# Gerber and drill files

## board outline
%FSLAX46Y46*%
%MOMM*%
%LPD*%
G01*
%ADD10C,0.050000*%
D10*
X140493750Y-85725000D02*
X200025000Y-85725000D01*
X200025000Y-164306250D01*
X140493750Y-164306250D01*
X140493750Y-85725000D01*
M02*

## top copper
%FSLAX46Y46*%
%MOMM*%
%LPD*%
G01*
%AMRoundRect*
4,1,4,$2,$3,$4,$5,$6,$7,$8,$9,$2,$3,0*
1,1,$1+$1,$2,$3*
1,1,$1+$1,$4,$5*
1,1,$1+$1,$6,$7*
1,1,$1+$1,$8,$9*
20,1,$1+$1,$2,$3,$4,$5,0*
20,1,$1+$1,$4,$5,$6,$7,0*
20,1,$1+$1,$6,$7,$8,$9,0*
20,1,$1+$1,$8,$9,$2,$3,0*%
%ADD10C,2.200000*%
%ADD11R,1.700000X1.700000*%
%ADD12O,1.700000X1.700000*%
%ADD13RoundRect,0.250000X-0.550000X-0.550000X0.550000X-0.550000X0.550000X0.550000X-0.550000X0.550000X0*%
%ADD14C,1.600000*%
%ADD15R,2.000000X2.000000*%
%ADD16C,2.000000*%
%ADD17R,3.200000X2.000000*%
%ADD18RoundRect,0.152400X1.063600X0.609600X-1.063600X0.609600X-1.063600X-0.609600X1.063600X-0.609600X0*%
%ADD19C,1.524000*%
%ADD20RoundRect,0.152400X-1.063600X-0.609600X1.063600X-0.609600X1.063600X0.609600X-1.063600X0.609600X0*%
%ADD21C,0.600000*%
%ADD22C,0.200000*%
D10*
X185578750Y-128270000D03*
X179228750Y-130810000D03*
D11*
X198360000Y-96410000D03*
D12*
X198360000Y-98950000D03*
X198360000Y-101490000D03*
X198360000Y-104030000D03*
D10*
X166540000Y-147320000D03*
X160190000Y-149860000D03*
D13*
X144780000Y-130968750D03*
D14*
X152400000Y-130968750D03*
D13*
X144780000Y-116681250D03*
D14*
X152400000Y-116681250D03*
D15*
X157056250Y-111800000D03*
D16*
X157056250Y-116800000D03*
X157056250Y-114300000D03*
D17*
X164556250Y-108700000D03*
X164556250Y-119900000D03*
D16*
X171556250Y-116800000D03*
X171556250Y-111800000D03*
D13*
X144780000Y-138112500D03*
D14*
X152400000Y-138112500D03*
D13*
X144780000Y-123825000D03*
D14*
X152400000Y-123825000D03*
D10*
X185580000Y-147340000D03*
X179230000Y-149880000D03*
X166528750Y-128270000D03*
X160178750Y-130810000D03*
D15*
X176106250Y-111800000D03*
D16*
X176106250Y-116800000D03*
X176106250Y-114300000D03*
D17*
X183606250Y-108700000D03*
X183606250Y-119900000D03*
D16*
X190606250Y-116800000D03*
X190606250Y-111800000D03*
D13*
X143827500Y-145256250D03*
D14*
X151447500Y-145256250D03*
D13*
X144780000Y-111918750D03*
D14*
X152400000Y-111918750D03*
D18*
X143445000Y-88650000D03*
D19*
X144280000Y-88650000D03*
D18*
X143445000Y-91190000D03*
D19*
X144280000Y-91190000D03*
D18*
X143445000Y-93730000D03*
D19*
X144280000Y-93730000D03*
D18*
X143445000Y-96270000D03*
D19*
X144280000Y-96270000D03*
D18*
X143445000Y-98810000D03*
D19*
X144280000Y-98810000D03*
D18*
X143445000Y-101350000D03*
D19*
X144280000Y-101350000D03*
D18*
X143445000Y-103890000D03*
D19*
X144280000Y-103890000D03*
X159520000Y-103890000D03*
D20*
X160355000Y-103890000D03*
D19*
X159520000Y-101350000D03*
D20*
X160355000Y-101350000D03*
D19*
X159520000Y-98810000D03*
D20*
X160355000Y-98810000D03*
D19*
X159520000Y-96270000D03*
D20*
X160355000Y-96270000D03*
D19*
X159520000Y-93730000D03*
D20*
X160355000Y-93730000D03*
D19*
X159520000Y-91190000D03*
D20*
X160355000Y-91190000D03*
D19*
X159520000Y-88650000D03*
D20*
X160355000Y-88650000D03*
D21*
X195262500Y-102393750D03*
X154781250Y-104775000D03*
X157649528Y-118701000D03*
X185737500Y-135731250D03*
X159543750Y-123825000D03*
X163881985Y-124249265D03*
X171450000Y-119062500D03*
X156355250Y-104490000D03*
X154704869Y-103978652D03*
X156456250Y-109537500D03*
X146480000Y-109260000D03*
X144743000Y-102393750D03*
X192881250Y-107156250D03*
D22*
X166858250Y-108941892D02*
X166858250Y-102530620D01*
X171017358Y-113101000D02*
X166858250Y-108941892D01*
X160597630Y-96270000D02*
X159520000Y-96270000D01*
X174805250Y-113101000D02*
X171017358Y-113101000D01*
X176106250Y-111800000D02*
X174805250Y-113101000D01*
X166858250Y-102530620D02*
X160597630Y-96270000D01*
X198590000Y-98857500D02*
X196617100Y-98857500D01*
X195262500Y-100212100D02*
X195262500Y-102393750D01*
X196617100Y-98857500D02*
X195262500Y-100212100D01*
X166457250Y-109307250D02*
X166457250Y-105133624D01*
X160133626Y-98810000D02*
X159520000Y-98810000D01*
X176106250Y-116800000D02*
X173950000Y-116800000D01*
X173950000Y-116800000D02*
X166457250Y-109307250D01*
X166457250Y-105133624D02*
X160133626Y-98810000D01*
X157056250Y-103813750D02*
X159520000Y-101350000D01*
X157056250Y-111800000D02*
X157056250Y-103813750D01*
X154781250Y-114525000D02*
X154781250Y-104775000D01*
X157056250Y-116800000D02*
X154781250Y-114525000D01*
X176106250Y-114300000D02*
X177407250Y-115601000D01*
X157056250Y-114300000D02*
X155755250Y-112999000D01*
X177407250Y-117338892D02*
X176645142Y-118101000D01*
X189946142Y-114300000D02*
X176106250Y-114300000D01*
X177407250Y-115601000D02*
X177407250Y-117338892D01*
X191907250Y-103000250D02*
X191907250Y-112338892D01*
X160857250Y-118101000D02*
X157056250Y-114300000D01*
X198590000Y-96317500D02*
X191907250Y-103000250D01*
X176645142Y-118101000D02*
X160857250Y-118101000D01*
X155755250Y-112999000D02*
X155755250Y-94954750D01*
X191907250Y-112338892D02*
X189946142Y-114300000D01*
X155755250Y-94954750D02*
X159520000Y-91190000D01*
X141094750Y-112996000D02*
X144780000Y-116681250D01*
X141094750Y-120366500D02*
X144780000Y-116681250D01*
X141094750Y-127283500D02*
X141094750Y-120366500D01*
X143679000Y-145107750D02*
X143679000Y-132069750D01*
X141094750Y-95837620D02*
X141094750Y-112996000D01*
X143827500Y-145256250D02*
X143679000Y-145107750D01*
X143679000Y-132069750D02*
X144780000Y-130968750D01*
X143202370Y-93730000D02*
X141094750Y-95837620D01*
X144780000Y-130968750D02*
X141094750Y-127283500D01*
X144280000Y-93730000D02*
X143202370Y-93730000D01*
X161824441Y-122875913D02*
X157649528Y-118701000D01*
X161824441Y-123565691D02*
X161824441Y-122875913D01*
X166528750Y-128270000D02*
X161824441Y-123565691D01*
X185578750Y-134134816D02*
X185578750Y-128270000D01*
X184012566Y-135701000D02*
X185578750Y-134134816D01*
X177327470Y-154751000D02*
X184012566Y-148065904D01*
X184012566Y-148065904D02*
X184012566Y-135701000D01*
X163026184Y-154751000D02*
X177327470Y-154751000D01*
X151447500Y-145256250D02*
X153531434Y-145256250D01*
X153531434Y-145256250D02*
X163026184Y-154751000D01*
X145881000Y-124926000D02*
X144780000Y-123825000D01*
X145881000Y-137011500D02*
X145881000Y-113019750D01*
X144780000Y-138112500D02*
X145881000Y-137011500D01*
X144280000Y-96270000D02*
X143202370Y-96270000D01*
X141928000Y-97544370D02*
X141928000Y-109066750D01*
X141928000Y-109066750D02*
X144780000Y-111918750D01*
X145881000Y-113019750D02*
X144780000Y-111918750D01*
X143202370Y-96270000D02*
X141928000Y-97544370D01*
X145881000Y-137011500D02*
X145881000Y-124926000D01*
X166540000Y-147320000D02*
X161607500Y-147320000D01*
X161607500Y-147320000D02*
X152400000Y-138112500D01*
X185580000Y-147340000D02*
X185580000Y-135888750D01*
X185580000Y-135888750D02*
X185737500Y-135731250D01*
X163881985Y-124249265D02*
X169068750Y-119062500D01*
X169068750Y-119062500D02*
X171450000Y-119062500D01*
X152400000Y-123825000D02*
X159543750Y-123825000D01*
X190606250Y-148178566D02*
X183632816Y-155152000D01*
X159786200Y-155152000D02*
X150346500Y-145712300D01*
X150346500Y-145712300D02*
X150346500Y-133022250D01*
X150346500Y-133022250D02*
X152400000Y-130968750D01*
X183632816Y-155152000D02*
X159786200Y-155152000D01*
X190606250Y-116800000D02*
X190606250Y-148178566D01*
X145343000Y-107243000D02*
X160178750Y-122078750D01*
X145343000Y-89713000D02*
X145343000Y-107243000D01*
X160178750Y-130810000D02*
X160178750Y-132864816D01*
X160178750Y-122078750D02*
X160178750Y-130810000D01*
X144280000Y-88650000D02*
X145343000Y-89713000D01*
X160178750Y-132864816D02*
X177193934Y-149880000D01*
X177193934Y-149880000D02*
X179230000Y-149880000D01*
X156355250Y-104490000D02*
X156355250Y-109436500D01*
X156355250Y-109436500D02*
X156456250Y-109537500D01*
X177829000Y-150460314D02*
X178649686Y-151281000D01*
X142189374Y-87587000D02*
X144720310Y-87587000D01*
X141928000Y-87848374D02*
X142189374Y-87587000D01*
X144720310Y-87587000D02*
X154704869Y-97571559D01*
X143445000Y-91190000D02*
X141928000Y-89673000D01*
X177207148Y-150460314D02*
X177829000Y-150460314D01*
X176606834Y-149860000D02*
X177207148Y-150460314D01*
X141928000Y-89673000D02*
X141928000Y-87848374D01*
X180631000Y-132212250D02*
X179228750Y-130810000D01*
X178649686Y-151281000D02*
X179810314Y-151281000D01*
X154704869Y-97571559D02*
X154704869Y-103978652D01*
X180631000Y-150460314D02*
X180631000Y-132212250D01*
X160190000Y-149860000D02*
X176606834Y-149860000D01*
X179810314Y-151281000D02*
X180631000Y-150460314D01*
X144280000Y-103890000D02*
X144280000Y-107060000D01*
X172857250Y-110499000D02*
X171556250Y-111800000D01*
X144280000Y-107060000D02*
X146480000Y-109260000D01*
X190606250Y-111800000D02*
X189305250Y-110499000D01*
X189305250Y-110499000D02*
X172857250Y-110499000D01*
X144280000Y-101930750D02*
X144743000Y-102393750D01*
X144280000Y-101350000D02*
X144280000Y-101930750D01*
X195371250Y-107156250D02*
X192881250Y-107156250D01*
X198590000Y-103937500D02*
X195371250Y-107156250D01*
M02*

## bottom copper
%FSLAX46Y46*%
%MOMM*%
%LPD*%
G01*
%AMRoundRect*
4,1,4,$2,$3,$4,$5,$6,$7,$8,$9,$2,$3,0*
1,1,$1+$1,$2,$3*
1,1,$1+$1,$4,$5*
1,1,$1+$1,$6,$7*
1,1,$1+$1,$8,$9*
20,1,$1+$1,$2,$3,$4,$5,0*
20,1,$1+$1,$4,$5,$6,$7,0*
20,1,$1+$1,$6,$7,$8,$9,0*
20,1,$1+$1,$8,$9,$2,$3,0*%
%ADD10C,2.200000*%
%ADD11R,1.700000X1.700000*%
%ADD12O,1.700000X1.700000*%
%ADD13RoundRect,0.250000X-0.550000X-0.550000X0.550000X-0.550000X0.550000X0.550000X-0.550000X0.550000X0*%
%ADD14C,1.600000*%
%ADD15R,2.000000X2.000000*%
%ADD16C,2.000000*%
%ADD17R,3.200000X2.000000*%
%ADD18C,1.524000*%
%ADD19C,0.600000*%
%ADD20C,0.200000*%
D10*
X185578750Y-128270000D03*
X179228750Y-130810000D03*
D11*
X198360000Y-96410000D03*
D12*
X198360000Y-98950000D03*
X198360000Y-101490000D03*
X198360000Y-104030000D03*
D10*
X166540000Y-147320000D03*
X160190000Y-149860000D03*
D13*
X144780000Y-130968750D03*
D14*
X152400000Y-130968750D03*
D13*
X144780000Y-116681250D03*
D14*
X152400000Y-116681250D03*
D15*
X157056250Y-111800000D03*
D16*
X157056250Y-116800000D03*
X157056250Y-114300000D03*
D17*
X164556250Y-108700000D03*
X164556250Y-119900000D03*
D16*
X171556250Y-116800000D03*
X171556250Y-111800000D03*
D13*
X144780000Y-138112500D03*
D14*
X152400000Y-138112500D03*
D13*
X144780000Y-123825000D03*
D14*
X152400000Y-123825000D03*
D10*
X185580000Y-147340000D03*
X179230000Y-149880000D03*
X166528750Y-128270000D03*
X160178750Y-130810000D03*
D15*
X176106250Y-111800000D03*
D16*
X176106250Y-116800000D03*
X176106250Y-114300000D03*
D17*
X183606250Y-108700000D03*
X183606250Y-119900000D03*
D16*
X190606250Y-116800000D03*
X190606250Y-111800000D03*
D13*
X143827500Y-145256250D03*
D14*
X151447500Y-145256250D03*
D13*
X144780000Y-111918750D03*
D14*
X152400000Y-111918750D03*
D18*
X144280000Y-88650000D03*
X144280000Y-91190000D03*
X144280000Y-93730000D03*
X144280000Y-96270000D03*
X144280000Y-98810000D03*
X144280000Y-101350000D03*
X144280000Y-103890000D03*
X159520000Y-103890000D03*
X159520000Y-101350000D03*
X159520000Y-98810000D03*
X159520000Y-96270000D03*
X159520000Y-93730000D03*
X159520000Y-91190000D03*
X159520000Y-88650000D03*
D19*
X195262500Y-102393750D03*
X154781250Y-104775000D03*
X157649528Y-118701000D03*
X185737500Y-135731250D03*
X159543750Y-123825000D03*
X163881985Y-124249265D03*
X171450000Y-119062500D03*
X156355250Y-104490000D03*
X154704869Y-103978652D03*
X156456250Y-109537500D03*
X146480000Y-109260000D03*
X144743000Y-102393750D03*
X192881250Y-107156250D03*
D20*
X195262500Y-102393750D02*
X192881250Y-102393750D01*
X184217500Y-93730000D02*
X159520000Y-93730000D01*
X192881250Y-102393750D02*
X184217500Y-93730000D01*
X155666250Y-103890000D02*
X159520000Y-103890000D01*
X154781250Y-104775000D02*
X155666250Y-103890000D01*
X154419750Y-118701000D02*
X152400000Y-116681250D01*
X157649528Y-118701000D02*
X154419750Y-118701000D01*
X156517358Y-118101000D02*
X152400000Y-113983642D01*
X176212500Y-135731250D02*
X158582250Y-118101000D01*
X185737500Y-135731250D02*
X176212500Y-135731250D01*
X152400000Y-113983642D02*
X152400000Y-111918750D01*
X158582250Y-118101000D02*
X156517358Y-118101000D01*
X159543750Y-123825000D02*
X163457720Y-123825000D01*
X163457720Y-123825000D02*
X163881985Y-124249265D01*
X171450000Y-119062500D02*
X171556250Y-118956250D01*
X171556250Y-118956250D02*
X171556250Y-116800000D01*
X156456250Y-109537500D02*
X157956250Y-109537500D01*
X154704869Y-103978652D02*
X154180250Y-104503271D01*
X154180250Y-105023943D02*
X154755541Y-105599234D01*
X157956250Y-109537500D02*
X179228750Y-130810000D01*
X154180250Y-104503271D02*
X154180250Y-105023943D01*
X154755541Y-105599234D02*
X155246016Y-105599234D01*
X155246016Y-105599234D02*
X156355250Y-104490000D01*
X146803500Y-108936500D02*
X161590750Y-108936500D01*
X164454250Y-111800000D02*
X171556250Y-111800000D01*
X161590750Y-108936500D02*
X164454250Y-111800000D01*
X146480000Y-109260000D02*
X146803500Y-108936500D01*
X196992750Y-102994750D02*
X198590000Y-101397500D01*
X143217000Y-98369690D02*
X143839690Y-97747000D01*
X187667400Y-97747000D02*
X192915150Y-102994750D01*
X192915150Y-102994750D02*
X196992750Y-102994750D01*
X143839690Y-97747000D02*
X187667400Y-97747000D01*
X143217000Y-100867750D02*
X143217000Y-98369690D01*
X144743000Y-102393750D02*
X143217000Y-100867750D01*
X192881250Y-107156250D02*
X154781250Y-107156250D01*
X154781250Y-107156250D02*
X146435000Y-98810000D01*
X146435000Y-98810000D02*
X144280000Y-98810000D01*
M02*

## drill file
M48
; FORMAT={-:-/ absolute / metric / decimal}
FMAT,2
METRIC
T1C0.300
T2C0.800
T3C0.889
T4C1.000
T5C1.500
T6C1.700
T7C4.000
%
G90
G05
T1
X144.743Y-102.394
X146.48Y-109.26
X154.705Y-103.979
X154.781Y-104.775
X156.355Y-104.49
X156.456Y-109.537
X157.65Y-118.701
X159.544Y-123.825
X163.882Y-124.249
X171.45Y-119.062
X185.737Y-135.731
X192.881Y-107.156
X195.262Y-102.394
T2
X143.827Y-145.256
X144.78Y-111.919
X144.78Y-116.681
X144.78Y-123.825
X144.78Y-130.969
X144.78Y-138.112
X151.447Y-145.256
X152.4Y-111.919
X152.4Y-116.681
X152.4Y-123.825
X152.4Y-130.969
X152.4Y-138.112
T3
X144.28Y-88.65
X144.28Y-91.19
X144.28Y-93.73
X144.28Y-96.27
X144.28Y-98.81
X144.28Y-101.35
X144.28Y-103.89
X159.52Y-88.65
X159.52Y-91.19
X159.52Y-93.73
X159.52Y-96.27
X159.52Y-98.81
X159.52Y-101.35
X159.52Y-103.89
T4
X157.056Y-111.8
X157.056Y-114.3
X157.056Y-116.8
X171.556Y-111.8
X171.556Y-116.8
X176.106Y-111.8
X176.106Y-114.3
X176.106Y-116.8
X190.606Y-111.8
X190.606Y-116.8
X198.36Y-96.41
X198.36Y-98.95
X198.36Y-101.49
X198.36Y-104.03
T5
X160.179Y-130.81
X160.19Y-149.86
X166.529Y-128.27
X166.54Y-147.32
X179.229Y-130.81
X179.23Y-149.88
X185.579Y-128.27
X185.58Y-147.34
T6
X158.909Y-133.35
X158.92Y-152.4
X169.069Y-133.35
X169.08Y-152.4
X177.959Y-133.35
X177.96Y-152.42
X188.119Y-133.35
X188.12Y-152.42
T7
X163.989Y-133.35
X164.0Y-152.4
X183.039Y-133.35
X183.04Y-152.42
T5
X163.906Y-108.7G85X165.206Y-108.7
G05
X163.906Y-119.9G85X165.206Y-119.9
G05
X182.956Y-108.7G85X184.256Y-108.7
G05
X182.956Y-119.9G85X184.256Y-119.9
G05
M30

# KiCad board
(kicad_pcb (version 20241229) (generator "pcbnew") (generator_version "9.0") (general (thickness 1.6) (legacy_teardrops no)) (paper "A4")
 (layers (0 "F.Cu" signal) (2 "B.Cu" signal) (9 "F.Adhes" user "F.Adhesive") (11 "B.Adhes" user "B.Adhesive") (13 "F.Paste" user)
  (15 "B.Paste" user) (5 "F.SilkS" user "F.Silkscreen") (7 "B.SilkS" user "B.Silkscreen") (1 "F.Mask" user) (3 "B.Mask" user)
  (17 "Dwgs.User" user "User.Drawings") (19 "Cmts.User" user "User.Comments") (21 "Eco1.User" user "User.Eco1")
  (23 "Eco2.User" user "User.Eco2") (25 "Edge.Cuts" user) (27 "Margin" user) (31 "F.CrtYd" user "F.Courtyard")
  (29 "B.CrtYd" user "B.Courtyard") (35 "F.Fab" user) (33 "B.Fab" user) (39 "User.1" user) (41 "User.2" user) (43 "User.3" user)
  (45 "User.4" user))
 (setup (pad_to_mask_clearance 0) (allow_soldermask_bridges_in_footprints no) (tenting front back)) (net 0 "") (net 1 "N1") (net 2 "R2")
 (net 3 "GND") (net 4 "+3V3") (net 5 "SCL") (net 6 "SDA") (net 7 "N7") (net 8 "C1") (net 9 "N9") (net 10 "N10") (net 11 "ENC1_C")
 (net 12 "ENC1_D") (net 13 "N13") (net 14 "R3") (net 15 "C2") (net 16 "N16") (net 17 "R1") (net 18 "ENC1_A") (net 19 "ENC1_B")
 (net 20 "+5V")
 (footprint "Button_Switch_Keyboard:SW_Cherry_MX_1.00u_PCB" (layer "F.Cu") (at 185.57875 128.27)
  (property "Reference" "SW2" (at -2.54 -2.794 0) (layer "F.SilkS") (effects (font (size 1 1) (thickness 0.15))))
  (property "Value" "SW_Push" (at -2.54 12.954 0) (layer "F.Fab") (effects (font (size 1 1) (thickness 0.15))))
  (pad "" np_thru_hole circle (at -7.62 5.08) (size 1.7 1.7) (drill 1.7) (layers "*.Cu" "*.Mask"))
  (pad "" np_thru_hole circle (at -2.54 5.08) (size 4 4) (drill 4) (layers "*.Cu" "*.Mask"))
  (pad "" np_thru_hole circle (at 2.54 5.08) (size 1.7 1.7) (drill 1.7) (layers "*.Cu" "*.Mask"))
  (pad "1" thru_hole circle (at 0 0) (size 2.2 2.2) (drill 1.5) (layers "*.Cu" "*.Mask") (remove_unused_layers no) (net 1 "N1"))
  (pad "2" thru_hole circle (at -6.35 2.54) (size 2.2 2.2) (drill 1.5) (layers "*.Cu" "*.Mask") (remove_unused_layers no) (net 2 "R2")))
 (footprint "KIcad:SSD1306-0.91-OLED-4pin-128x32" (layer "F.Cu") (at 161.86 94.22)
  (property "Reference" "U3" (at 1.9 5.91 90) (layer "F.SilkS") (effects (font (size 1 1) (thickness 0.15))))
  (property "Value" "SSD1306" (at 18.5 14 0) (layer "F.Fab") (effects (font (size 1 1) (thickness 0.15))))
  (pad "1" thru_hole rect (at 36.5 2.19) (size 1.7 1.7) (drill 1) (layers "*.Cu" "*.Mask") (remove_unused_layers no) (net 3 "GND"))
  (pad "2" thru_hole oval (at 36.5 4.73) (size 1.7 1.7) (drill 1) (layers "*.Cu" "*.Mask") (remove_unused_layers no) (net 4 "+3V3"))
  (pad "3" thru_hole oval (at 36.5 7.27) (size 1.7 1.7) (drill 1) (layers "*.Cu" "*.Mask") (remove_unused_layers no) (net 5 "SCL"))
  (pad "4" thru_hole oval (at 36.5 9.81) (size 1.7 1.7) (drill 1) (layers "*.Cu" "*.Mask") (remove_unused_layers no) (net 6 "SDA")))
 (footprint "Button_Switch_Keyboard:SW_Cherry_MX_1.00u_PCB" (layer "F.Cu") (at 166.54 147.32)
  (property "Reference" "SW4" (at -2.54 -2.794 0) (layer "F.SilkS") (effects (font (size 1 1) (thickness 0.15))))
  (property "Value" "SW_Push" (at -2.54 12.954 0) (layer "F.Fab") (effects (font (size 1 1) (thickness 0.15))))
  (pad "" np_thru_hole circle (at -7.62 5.08) (size 1.7 1.7) (drill 1.7) (layers "*.Cu" "*.Mask"))
  (pad "" np_thru_hole circle (at -2.54 5.08) (size 4 4) (drill 4) (layers "*.Cu" "*.Mask"))
  (pad "" np_thru_hole circle (at 2.54 5.08) (size 1.7 1.7) (drill 1.7) (layers "*.Cu" "*.Mask"))
  (pad "1" thru_hole circle (at 0 0) (size 2.2 2.2) (drill 1.5) (layers "*.Cu" "*.Mask") (remove_unused_layers no) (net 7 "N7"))
  (pad "2" thru_hole circle (at -6.35 2.54) (size 2.2 2.2) (drill 1.5) (layers "*.Cu" "*.Mask") (remove_unused_layers no) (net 2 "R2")))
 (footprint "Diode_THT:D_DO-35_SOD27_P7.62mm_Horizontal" (layer "F.Cu") (at 144.78 130.96875)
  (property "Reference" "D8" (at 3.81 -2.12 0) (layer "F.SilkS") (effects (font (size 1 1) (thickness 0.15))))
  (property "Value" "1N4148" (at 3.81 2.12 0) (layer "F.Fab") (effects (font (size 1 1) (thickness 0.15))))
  (pad "1" thru_hole roundrect (at 0 0) (size 1.6 1.6) (drill 0.8) (layers "*.Cu" "*.Mask") (remove_unused_layers no)
   (roundrect_rratio 0.15625) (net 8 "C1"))
  (pad "2" thru_hole circle (at 7.62 0) (size 1.6 1.6) (drill 0.8) (layers "*.Cu" "*.Mask") (remove_unused_layers no) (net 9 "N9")))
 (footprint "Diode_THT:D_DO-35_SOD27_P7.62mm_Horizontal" (layer "F.Cu") (at 144.78 116.68125)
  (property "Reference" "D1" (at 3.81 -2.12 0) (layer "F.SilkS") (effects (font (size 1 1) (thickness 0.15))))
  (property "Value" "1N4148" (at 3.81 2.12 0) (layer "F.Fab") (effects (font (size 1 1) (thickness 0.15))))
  (pad "1" thru_hole roundrect (at 0 0) (size 1.6 1.6) (drill 0.8) (layers "*.Cu" "*.Mask") (remove_unused_layers no)
   (roundrect_rratio 0.15625) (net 8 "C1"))
  (pad "2" thru_hole circle (at 7.62 0) (size 1.6 1.6) (drill 0.8) (layers "*.Cu" "*.Mask") (remove_unused_layers no) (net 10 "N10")))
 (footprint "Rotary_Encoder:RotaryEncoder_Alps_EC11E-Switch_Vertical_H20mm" (layer "F.Cu") (at 157.05625 111.8)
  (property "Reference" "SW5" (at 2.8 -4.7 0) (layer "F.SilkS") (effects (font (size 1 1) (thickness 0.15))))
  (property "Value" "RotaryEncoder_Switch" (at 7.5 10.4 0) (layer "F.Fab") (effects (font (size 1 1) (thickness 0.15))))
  (pad "A" thru_hole rect (at 0 0) (size 2 2) (drill 1) (layers "*.Cu" "*.Mask") (remove_unused_layers no) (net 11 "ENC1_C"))
  (pad "B" thru_hole circle (at 0 5) (size 2 2) (drill 1) (layers "*.Cu" "*.Mask") (remove_unused_layers no) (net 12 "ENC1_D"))
  (pad "C" thru_hole circle (at 0 2.5) (size 2 2) (drill 1) (layers "*.Cu" "*.Mask") (remove_unused_layers no) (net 3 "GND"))
  (pad "MP" thru_hole rect (at 7.5 -3.1) (size 3.2 2) (drill oval 2.8 1.5) (layers "*.Cu" "*.Mask") (remove_unused_layers no))
  (pad "MP" thru_hole rect (at 7.5 8.1) (size 3.2 2) (drill oval 2.8 1.5) (layers "*.Cu" "*.Mask") (remove_unused_layers no))
  (pad "S1" thru_hole circle (at 14.5 5) (size 2 2) (drill 1) (layers "*.Cu" "*.Mask") (remove_unused_layers no) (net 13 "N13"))
  (pad "S2" thru_hole circle (at 14.5 0) (size 2 2) (drill 1) (layers "*.Cu" "*.Mask") (remove_unused_layers no) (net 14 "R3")))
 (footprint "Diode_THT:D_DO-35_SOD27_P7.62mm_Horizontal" (layer "F.Cu") (at 144.78 138.1125)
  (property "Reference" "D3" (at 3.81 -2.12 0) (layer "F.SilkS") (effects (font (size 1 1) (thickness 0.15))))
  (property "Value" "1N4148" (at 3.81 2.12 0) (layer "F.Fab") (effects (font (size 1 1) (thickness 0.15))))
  (pad "1" thru_hole roundrect (at 0 0) (size 1.6 1.6) (drill 0.8) (layers "*.Cu" "*.Mask") (remove_unused_layers no)
   (roundrect_rratio 0.15625) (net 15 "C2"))
  (pad "2" thru_hole circle (at 7.62 0) (size 1.6 1.6) (drill 0.8) (layers "*.Cu" "*.Mask") (remove_unused_layers no) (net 7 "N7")))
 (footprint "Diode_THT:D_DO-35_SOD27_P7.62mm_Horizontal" (layer "F.Cu") (at 144.78 123.825)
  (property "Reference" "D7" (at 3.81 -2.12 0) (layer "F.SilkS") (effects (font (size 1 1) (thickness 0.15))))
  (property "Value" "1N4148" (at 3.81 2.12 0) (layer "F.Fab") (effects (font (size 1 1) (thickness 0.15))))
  (pad "1" thru_hole roundrect (at 0 0) (size 1.6 1.6) (drill 0.8) (layers "*.Cu" "*.Mask") (remove_unused_layers no)
   (roundrect_rratio 0.15625) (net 15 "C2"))
  (pad "2" thru_hole circle (at 7.62 0) (size 1.6 1.6) (drill 0.8) (layers "*.Cu" "*.Mask") (remove_unused_layers no) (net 13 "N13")))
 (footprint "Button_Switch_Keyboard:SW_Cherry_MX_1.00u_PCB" (layer "F.Cu") (at 185.58 147.34)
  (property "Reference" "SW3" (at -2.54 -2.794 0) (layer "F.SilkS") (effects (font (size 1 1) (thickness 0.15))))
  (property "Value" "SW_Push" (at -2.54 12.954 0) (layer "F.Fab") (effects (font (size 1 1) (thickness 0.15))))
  (pad "" np_thru_hole circle (at -7.62 5.08) (size 1.7 1.7) (drill 1.7) (layers "*.Cu" "*.Mask"))
  (pad "" np_thru_hole circle (at -2.54 5.08) (size 4 4) (drill 4) (layers "*.Cu" "*.Mask"))
  (pad "" np_thru_hole circle (at 2.54 5.08) (size 1.7 1.7) (drill 1.7) (layers "*.Cu" "*.Mask"))
  (pad "1" thru_hole circle (at 0 0) (size 2.2 2.2) (drill 1.5) (layers "*.Cu" "*.Mask") (remove_unused_layers no) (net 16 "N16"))
  (pad "2" thru_hole circle (at -6.35 2.54) (size 2.2 2.2) (drill 1.5) (layers "*.Cu" "*.Mask") (remove_unused_layers no) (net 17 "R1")))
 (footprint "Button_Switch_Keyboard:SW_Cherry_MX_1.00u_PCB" (layer "F.Cu") (at 166.52875 128.27)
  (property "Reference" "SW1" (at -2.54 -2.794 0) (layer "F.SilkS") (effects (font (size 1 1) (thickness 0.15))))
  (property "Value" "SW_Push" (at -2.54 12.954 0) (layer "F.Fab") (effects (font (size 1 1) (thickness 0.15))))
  (pad "" np_thru_hole circle (at -7.62 5.08) (size 1.7 1.7) (drill 1.7) (layers "*.Cu" "*.Mask"))
  (pad "" np_thru_hole circle (at -2.54 5.08) (size 4 4) (drill 4) (layers "*.Cu" "*.Mask"))
  (pad "" np_thru_hole circle (at 2.54 5.08) (size 1.7 1.7) (drill 1.7) (layers "*.Cu" "*.Mask"))
  (pad "1" thru_hole circle (at 0 0) (size 2.2 2.2) (drill 1.5) (layers "*.Cu" "*.Mask") (remove_unused_layers no) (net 10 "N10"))
  (pad "2" thru_hole circle (at -6.35 2.54) (size 2.2 2.2) (drill 1.5) (layers "*.Cu" "*.Mask") (remove_unused_layers no) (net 17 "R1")))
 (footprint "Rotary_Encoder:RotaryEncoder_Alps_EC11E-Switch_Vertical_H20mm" (layer "F.Cu") (at 176.10625 111.8)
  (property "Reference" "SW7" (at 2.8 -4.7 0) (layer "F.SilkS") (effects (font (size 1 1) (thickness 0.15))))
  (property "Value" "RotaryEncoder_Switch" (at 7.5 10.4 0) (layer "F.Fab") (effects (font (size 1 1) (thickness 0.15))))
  (pad "A" thru_hole rect (at 0 0) (size 2 2) (drill 1) (layers "*.Cu" "*.Mask") (remove_unused_layers no) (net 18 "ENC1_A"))
  (pad "B" thru_hole circle (at 0 5) (size 2 2) (drill 1) (layers "*.Cu" "*.Mask") (remove_unused_layers no) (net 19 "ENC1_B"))
  (pad "C" thru_hole circle (at 0 2.5) (size 2 2) (drill 1) (layers "*.Cu" "*.Mask") (remove_unused_layers no) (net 3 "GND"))
  (pad "MP" thru_hole rect (at 7.5 -3.1) (size 3.2 2) (drill oval 2.8 1.5) (layers "*.Cu" "*.Mask") (remove_unused_layers no))
  (pad "MP" thru_hole rect (at 7.5 8.1) (size 3.2 2) (drill oval 2.8 1.5) (layers "*.Cu" "*.Mask") (remove_unused_layers no))
  (pad "S1" thru_hole circle (at 14.5 5) (size 2 2) (drill 1) (layers "*.Cu" "*.Mask") (remove_unused_layers no) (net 9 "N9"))
  (pad "S2" thru_hole circle (at 14.5 0) (size 2 2) (drill 1) (layers "*.Cu" "*.Mask") (remove_unused_layers no) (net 14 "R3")))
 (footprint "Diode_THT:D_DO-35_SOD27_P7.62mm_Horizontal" (layer "F.Cu") (at 143.8275 145.25625)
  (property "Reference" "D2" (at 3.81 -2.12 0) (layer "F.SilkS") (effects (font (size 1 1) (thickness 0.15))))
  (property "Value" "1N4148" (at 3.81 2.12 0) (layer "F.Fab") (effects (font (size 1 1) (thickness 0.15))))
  (pad "1" thru_hole roundrect (at 0 0) (size 1.6 1.6) (drill 0.8) (layers "*.Cu" "*.Mask") (remove_unused_layers no)
   (roundrect_rratio 0.15625) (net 8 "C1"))
  (pad "2" thru_hole circle (at 7.62 0) (size 1.6 1.6) (drill 0.8) (layers "*.Cu" "*.Mask") (remove_unused_layers no) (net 1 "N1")))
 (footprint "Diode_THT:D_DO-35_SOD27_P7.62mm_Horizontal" (layer "F.Cu") (at 144.78 111.91875)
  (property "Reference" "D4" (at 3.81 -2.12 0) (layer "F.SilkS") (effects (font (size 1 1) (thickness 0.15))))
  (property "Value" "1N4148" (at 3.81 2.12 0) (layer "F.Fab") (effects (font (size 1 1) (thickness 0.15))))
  (pad "1" thru_hole roundrect (at 0 0) (size 1.6 1.6) (drill 0.8) (layers "*.Cu" "*.Mask") (remove_unused_layers no)
   (roundrect_rratio 0.15625) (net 15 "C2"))
  (pad "2" thru_hole circle (at 7.62 0) (size 1.6 1.6) (drill 0.8) (layers "*.Cu" "*.Mask") (remove_unused_layers no) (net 16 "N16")))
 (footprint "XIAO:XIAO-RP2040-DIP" (layer "F.Cu") (at 151.9 96.27)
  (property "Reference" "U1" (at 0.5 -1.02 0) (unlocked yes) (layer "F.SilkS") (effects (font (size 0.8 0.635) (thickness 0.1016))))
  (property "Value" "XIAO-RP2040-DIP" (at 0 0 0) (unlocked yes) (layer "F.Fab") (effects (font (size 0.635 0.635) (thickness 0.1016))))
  (pad "1" smd roundrect (at -8.455 -7.62 180) (size 2.432 1.524) (layers "F.Cu" "F.Mask") (roundrect_rratio 0.1) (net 17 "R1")
   (thermal_bridge_angle 45))
  (pad "1" thru_hole circle (at -7.62 -7.62 180) (size 1.524 1.524) (drill 0.889) (layers "*.Cu" "*.Mask") (remove_unused_layers no)
   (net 17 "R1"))
  (pad "2" smd roundrect (at -8.455 -5.08 180) (size 2.432 1.524) (layers "F.Cu" "F.Mask") (roundrect_rratio 0.1) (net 2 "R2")
   (thermal_bridge_angle 45))
  (pad "2" thru_hole circle (at -7.62 -5.08 180) (size 1.524 1.524) (drill 0.889) (layers "*.Cu" "*.Mask") (remove_unused_layers no)
   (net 2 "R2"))
  (pad "3" smd roundrect (at -8.455 -2.54 180) (size 2.432 1.524) (layers "F.Cu" "F.Mask") (roundrect_rratio 0.1) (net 8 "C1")
   (thermal_bridge_angle 45))
  (pad "3" thru_hole circle (at -7.62 -2.54 180) (size 1.524 1.524) (drill 0.889) (layers "*.Cu" "*.Mask") (remove_unused_layers no)
   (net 8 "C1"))
  (pad "4" smd roundrect (at -8.455 0 180) (size 2.432 1.524) (layers "F.Cu" "F.Mask") (roundrect_rratio 0.1) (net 15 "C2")
   (thermal_bridge_angle 45))
  (pad "4" thru_hole circle (at -7.62 0 180) (size 1.524 1.524) (drill 0.889) (layers "*.Cu" "*.Mask") (remove_unused_layers no)
   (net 15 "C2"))
  (pad "5" smd roundrect (at -8.455 2.54 180) (size 2.432 1.524) (layers "F.Cu" "F.Mask") (roundrect_rratio 0.1) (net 6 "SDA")
   (thermal_bridge_angle 45))
  (pad "5" thru_hole circle (at -7.62 2.54 180) (size 1.524 1.524) (drill 0.889) (layers "*.Cu" "*.Mask") (remove_unused_layers no)
   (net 6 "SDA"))
  (pad "6" smd roundrect (at -8.455 5.08 180) (size 2.432 1.524) (layers "F.Cu" "F.Mask") (roundrect_rratio 0.1) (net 5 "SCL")
   (thermal_bridge_angle 45))
  (pad "6" thru_hole circle (at -7.62 5.08 180) (size 1.524 1.524) (drill 0.889) (layers "*.Cu" "*.Mask") (remove_unused_layers no)
   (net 5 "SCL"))
  (pad "7" smd roundrect (at -8.455 7.62 180) (size 2.432 1.524) (layers "F.Cu" "F.Mask") (roundrect_rratio 0.1) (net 14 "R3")
   (thermal_bridge_angle 45))
  (pad "7" thru_hole circle (at -7.62 7.62 180) (size 1.524 1.524) (drill 0.889) (layers "*.Cu" "*.Mask") (remove_unused_layers no)
   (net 14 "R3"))
  (pad "8" thru_hole circle (at 7.62 7.62) (size 1.524 1.524) (drill 0.889) (layers "*.Cu" "*.Mask") (remove_unused_layers no)
   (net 12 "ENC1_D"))
  (pad "8" smd roundrect (at 8.455 7.62) (size 2.432 1.524) (layers "F.Cu" "F.Mask") (roundrect_rratio 0.1) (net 12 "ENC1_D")
   (thermal_bridge_angle 45))
  (pad "9" thru_hole circle (at 7.62 5.08) (size 1.524 1.524) (drill 0.889) (layers "*.Cu" "*.Mask") (remove_unused_layers no)
   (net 11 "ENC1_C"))
  (pad "9" smd roundrect (at 8.455 5.08) (size 2.432 1.524) (layers "F.Cu" "F.Mask") (roundrect_rratio 0.1) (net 11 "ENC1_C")
   (thermal_bridge_angle 45))
  (pad "10" thru_hole circle (at 7.62 2.54) (size 1.524 1.524) (drill 0.889) (layers "*.Cu" "*.Mask") (remove_unused_layers no)
   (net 19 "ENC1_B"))
  (pad "10" smd roundrect (at 8.455 2.54) (size 2.432 1.524) (layers "F.Cu" "F.Mask") (roundrect_rratio 0.1) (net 19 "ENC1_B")
   (thermal_bridge_angle 45))
  (pad "11" thru_hole circle (at 7.62 0) (size 1.524 1.524) (drill 0.889) (layers "*.Cu" "*.Mask") (remove_unused_layers no)
   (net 18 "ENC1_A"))
  (pad "11" smd roundrect (at 8.455 0) (size 2.432 1.524) (layers "F.Cu" "F.Mask") (roundrect_rratio 0.1) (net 18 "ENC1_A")
   (thermal_bridge_angle 45))
  (pad "12" thru_hole circle (at 7.62 -2.54) (size 1.524 1.524) (drill 0.889) (layers "*.Cu" "*.Mask") (remove_unused_layers no)
   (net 4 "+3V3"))
  (pad "12" smd roundrect (at 8.455 -2.54) (size 2.432 1.524) (layers "F.Cu" "F.Mask") (roundrect_rratio 0.1) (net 4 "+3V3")
   (thermal_bridge_angle 45))
  (pad "13" thru_hole circle (at 7.62 -5.08) (size 1.524 1.524) (drill 0.889) (layers "*.Cu" "*.Mask") (remove_unused_layers no)
   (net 3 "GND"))
  (pad "13" smd roundrect (at 8.455 -5.08) (size 2.432 1.524) (layers "F.Cu" "F.Mask") (roundrect_rratio 0.1) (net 3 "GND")
   (thermal_bridge_angle 45))
  (pad "14" thru_hole circle (at 7.62 -7.62) (size 1.524 1.524) (drill 0.889) (layers "*.Cu" "*.Mask") (remove_unused_layers no)
   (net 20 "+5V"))
  (pad "14" smd roundrect (at 8.455 -7.62) (size 2.432 1.524) (layers "F.Cu" "F.Mask") (roundrect_rratio 0.1) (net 20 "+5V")
   (thermal_bridge_angle 45)))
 (gr_rect (start 140.49375 85.725) (end 200.025 164.30625) (stroke (width 0.05) (type default)) (fill no) (layer "Edge.Cuts"))
 (segment (start 166.85825 108.941892) (end 166.85825 102.53062) (width 0.2) (layer "F.Cu") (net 18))
 (segment (start 171.017358 113.101) (end 166.85825 108.941892) (width 0.2) (layer "F.Cu") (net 18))
 (segment (start 160.59763 96.27) (end 159.52 96.27) (width 0.2) (layer "F.Cu") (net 18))
 (segment (start 174.80525 113.101) (end 171.017358 113.101) (width 0.2) (layer "F.Cu") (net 18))
 (segment (start 176.10625 111.8) (end 174.80525 113.101) (width 0.2) (layer "F.Cu") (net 18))
 (segment (start 166.85825 102.53062) (end 160.59763 96.27) (width 0.2) (layer "F.Cu") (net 18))
 (segment (start 198.59 98.8575) (end 196.6171 98.8575) (width 0.2) (layer "F.Cu") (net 4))
 (segment (start 195.2625 100.2121) (end 195.2625 102.39375) (width 0.2) (layer "F.Cu") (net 4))
 (segment (start 196.6171 98.8575) (end 195.2625 100.2121) (width 0.2) (layer "F.Cu") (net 4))
 (via (at 195.2625 102.39375) (size 0.6) (drill 0.3) (layers "F.Cu" "B.Cu") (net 4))
 (segment (start 195.2625 102.39375) (end 192.88125 102.39375) (width 0.2) (layer "B.Cu") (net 4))
 (segment (start 184.2175 93.73) (end 159.52 93.73) (width 0.2) (layer "B.Cu") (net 4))
 (segment (start 192.88125 102.39375) (end 184.2175 93.73) (width 0.2) (layer "B.Cu") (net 4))
 (segment (start 166.45725 109.30725) (end 166.45725 105.133624) (width 0.2) (layer "F.Cu") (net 19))
 (segment (start 160.133626 98.81) (end 159.52 98.81) (width 0.2) (layer "F.Cu") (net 19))
 (segment (start 176.10625 116.8) (end 173.95 116.8) (width 0.2) (layer "F.Cu") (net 19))
 (segment (start 173.95 116.8) (end 166.45725 109.30725) (width 0.2) (layer "F.Cu") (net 19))
 (segment (start 166.45725 105.133624) (end 160.133626 98.81) (width 0.2) (layer "F.Cu") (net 19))
 (segment (start 157.05625 103.81375) (end 159.52 101.35) (width 0.2) (layer "F.Cu") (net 11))
 (segment (start 157.05625 111.8) (end 157.05625 103.81375) (width 0.2) (layer "F.Cu") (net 11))
 (segment (start 154.78125 114.525) (end 154.78125 104.775) (width 0.2) (layer "F.Cu") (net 12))
 (segment (start 157.05625 116.8) (end 154.78125 114.525) (width 0.2) (layer "F.Cu") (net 12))
 (via (at 154.78125 104.775) (size 0.6) (drill 0.3) (layers "F.Cu" "B.Cu") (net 12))
 (segment (start 155.66625 103.89) (end 159.52 103.89) (width 0.2) (layer "B.Cu") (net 12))
 (segment (start 154.78125 104.775) (end 155.66625 103.89) (width 0.2) (layer "B.Cu") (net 12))
 (segment (start 176.10625 114.3) (end 177.40725 115.601) (width 0.2) (layer "F.Cu") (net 3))
 (segment (start 157.05625 114.3) (end 155.75525 112.999) (width 0.2) (layer "F.Cu") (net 3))
 (segment (start 177.40725 117.338892) (end 176.645142 118.101) (width 0.2) (layer "F.Cu") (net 3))
 (segment (start 189.946142 114.3) (end 176.10625 114.3) (width 0.2) (layer "F.Cu") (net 3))
 (segment (start 177.40725 115.601) (end 177.40725 117.338892) (width 0.2) (layer "F.Cu") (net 3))
 (segment (start 191.90725 103.00025) (end 191.90725 112.338892) (width 0.2) (layer "F.Cu") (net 3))
 (segment (start 160.85725 118.101) (end 157.05625 114.3) (width 0.2) (layer "F.Cu") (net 3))
 (segment (start 198.59 96.3175) (end 191.90725 103.00025) (width 0.2) (layer "F.Cu") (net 3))
 (segment (start 176.645142 118.101) (end 160.85725 118.101) (width 0.2) (layer "F.Cu") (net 3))
 (segment (start 155.75525 112.999) (end 155.75525 94.95475) (width 0.2) (layer "F.Cu") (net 3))
 (segment (start 191.90725 112.338892) (end 189.946142 114.3) (width 0.2) (layer "F.Cu") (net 3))
 (segment (start 155.75525 94.95475) (end 159.52 91.19) (width 0.2) (layer "F.Cu") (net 3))
 (segment (start 141.09475 112.996) (end 144.78 116.68125) (width 0.2) (layer "F.Cu") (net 8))
 (segment (start 141.09475 120.3665) (end 144.78 116.68125) (width 0.2) (layer "F.Cu") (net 8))
 (segment (start 141.09475 127.2835) (end 141.09475 120.3665) (width 0.2) (layer "F.Cu") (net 8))
 (segment (start 143.679 145.10775) (end 143.679 132.06975) (width 0.2) (layer "F.Cu") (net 8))
 (segment (start 141.09475 95.83762) (end 141.09475 112.996) (width 0.2) (layer "F.Cu") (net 8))
 (segment (start 143.8275 145.25625) (end 143.679 145.10775) (width 0.2) (layer "F.Cu") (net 8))
 (segment (start 143.679 132.06975) (end 144.78 130.96875) (width 0.2) (layer "F.Cu") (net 8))
 (segment (start 143.20237 93.73) (end 141.09475 95.83762) (width 0.2) (layer "F.Cu") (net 8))
 (segment (start 144.78 130.96875) (end 141.09475 127.2835) (width 0.2) (layer "F.Cu") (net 8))
 (segment (start 144.28 93.73) (end 143.20237 93.73) (width 0.2) (layer "F.Cu") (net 8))
 (segment (start 161.824441 122.875913) (end 157.649528 118.701) (width 0.2) (layer "F.Cu") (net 10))
 (segment (start 161.824441 123.565691) (end 161.824441 122.875913) (width 0.2) (layer "F.Cu") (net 10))
 (segment (start 166.52875 128.27) (end 161.824441 123.565691) (width 0.2) (layer "F.Cu") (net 10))
 (via (at 157.649528 118.701) (size 0.6) (drill 0.3) (layers "F.Cu" "B.Cu") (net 10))
 (segment (start 154.41975 118.701) (end 152.4 116.68125) (width 0.2) (layer "B.Cu") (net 10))
 (segment (start 157.649528 118.701) (end 154.41975 118.701) (width 0.2) (layer "B.Cu") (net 10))
 (segment (start 185.57875 134.134816) (end 185.57875 128.27) (width 0.2) (layer "F.Cu") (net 1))
 (segment (start 184.012566 135.701) (end 185.57875 134.134816) (width 0.2) (layer "F.Cu") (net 1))
 (segment (start 177.32747 154.751) (end 184.012566 148.065904) (width 0.2) (layer "F.Cu") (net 1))
 (segment (start 184.012566 148.065904) (end 184.012566 135.701) (width 0.2) (layer "F.Cu") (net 1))
 (segment (start 163.026184 154.751) (end 177.32747 154.751) (width 0.2) (layer "F.Cu") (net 1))
 (segment (start 151.4475 145.25625) (end 153.531434 145.25625) (width 0.2) (layer "F.Cu") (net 1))
 (segment (start 153.531434 145.25625) (end 163.026184 154.751) (width 0.2) (layer "F.Cu") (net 1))
 (segment (start 145.881 124.926) (end 144.78 123.825) (width 0.2) (layer "F.Cu") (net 15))
 (segment (start 145.881 137.0115) (end 145.881 113.01975) (width 0.2) (layer "F.Cu") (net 15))
 (segment (start 144.78 138.1125) (end 145.881 137.0115) (width 0.2) (layer "F.Cu") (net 15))
 (segment (start 144.28 96.27) (end 143.20237 96.27) (width 0.2) (layer "F.Cu") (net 15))
 (segment (start 141.928 97.54437) (end 141.928 109.06675) (width 0.2) (layer "F.Cu") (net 15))
 (segment (start 141.928 109.06675) (end 144.78 111.91875) (width 0.2) (layer "F.Cu") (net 15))
 (segment (start 145.881 113.01975) (end 144.78 111.91875) (width 0.2) (layer "F.Cu") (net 15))
 (segment (start 143.20237 96.27) (end 141.928 97.54437) (width 0.2) (layer "F.Cu") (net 15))
 (segment (start 145.881 137.0115) (end 145.881 124.926) (width 0.2) (layer "F.Cu") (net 15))
 (segment (start 166.54 147.32) (end 161.6075 147.32) (width 0.2) (layer "F.Cu") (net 7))
 (segment (start 161.6075 147.32) (end 152.4 138.1125) (width 0.2) (layer "F.Cu") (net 7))
 (segment (start 185.58 147.34) (end 185.58 135.88875) (width 0.2) (layer "F.Cu") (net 16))
 (segment (start 185.58 135.88875) (end 185.7375 135.73125) (width 0.2) (layer "F.Cu") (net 16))
 (via (at 185.7375 135.73125) (size 0.6) (drill 0.3) (layers "F.Cu" "B.Cu") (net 16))
 (segment (start 156.517358 118.101) (end 152.4 113.983642) (width 0.2) (layer "B.Cu") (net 16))
 (segment (start 176.2125 135.73125) (end 158.58225 118.101) (width 0.2) (layer "B.Cu") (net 16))
 (segment (start 185.7375 135.73125) (end 176.2125 135.73125) (width 0.2) (layer "B.Cu") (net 16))
 (segment (start 152.4 113.983642) (end 152.4 111.91875) (width 0.2) (layer "B.Cu") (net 16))
 (segment (start 158.58225 118.101) (end 156.517358 118.101) (width 0.2) (layer "B.Cu") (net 16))
 (segment (start 163.881985 124.249265) (end 169.06875 119.0625) (width 0.2) (layer "F.Cu") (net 13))
 (segment (start 169.06875 119.0625) (end 171.45 119.0625) (width 0.2) (layer "F.Cu") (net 13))
 (segment (start 152.4 123.825) (end 159.54375 123.825) (width 0.2) (layer "F.Cu") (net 13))
 (via (at 159.54375 123.825) (size 0.6) (drill 0.3) (layers "F.Cu" "B.Cu") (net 13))
 (via (at 163.881985 124.249265) (size 0.6) (drill 0.3) (layers "F.Cu" "B.Cu") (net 13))
 (via (at 171.45 119.0625) (size 0.6) (drill 0.3) (layers "F.Cu" "B.Cu") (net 13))
 (segment (start 159.54375 123.825) (end 163.45772 123.825) (width 0.2) (layer "B.Cu") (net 13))
 (segment (start 163.45772 123.825) (end 163.881985 124.249265) (width 0.2) (layer "B.Cu") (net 13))
 (segment (start 171.45 119.0625) (end 171.55625 118.95625) (width 0.2) (layer "B.Cu") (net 13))
 (segment (start 171.55625 118.95625) (end 171.55625 116.8) (width 0.2) (layer "B.Cu") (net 13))
 (segment (start 190.60625 148.178566) (end 183.632816 155.152) (width 0.2) (layer "F.Cu") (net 9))
 (segment (start 159.7862 155.152) (end 150.3465 145.7123) (width 0.2) (layer "F.Cu") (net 9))
 (segment (start 150.3465 145.7123) (end 150.3465 133.02225) (width 0.2) (layer "F.Cu") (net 9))
 (segment (start 150.3465 133.02225) (end 152.4 130.96875) (width 0.2) (layer "F.Cu") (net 9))
 (segment (start 183.632816 155.152) (end 159.7862 155.152) (width 0.2) (layer "F.Cu") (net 9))
 (segment (start 190.60625 116.8) (end 190.60625 148.178566) (width 0.2) (layer "F.Cu") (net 9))
 (segment (start 145.343 107.243) (end 160.17875 122.07875) (width 0.2) (layer "F.Cu") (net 17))
 (segment (start 145.343 89.713) (end 145.343 107.243) (width 0.2) (layer "F.Cu") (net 17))
 (segment (start 160.17875 130.81) (end 160.17875 132.864816) (width 0.2) (layer "F.Cu") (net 17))
 (segment (start 160.17875 122.07875) (end 160.17875 130.81) (width 0.2) (layer "F.Cu") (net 17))
 (segment (start 144.28 88.65) (end 145.343 89.713) (width 0.2) (layer "F.Cu") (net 17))
 (segment (start 160.17875 132.864816) (end 177.193934 149.88) (width 0.2) (layer "F.Cu") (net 17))
 (segment (start 177.193934 149.88) (end 179.23 149.88) (width 0.2) (layer "F.Cu") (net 17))
 (segment (start 156.35525 104.49) (end 156.35525 109.4365) (width 0.2) (layer "F.Cu") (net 2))
 (segment (start 156.35525 109.4365) (end 156.45625 109.5375) (width 0.2) (layer "F.Cu") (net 2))
 (segment (start 177.829 150.460314) (end 178.649686 151.281) (width 0.2) (layer "F.Cu") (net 2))
 (segment (start 142.189374 87.587) (end 144.72031 87.587) (width 0.2) (layer "F.Cu") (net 2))
 (segment (start 141.928 87.848374) (end 142.189374 87.587) (width 0.2) (layer "F.Cu") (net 2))
 (segment (start 144.72031 87.587) (end 154.704869 97.571559) (width 0.2) (layer "F.Cu") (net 2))
 (segment (start 143.445 91.19) (end 141.928 89.673) (width 0.2) (layer "F.Cu") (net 2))
 (segment (start 177.207148 150.460314) (end 177.829 150.460314) (width 0.2) (layer "F.Cu") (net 2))
 (segment (start 176.606834 149.86) (end 177.207148 150.460314) (width 0.2) (layer "F.Cu") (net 2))
 (segment (start 141.928 89.673) (end 141.928 87.848374) (width 0.2) (layer "F.Cu") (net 2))
 (segment (start 180.631 132.21225) (end 179.22875 130.81) (width 0.2) (layer "F.Cu") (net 2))
 (segment (start 178.649686 151.281) (end 179.810314 151.281) (width 0.2) (layer "F.Cu") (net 2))
 (segment (start 154.704869 97.571559) (end 154.704869 103.978652) (width 0.2) (layer "F.Cu") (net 2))
 (segment (start 180.631 150.460314) (end 180.631 132.21225) (width 0.2) (layer "F.Cu") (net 2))
 (segment (start 160.19 149.86) (end 176.606834 149.86) (width 0.2) (layer "F.Cu") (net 2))
 (segment (start 179.810314 151.281) (end 180.631 150.460314) (width 0.2) (layer "F.Cu") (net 2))
 (via (at 156.35525 104.49) (size 0.6) (drill 0.3) (layers "F.Cu" "B.Cu") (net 2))
 (via (at 154.704869 103.978652) (size 0.6) (drill 0.3) (layers "F.Cu" "B.Cu") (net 2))
 (via (at 156.45625 109.5375) (size 0.6) (drill 0.3) (layers "F.Cu" "B.Cu") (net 2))
 (segment (start 156.45625 109.5375) (end 157.95625 109.5375) (width 0.2) (layer "B.Cu") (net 2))
 (segment (start 154.704869 103.978652) (end 154.18025 104.503271) (width 0.2) (layer "B.Cu") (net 2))
 (segment (start 154.18025 105.023943) (end 154.755541 105.599234) (width 0.2) (layer "B.Cu") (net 2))
 (segment (start 157.95625 109.5375) (end 179.22875 130.81) (width 0.2) (layer "B.Cu") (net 2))
 (segment (start 154.18025 104.503271) (end 154.18025 105.023943) (width 0.2) (layer "B.Cu") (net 2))
 (segment (start 154.755541 105.599234) (end 155.246016 105.599234) (width 0.2) (layer "B.Cu") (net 2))
 (segment (start 155.246016 105.599234) (end 156.35525 104.49) (width 0.2) (layer "B.Cu") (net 2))
 (segment (start 144.28 103.89) (end 144.28 107.06) (width 0.2) (layer "F.Cu") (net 14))
 (segment (start 172.85725 110.499) (end 171.55625 111.8) (width 0.2) (layer "F.Cu") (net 14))
 (segment (start 144.28 107.06) (end 146.48 109.26) (width 0.2) (layer "F.Cu") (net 14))
 (segment (start 190.60625 111.8) (end 189.30525 110.499) (width 0.2) (layer "F.Cu") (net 14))
 (segment (start 189.30525 110.499) (end 172.85725 110.499) (width 0.2) (layer "F.Cu") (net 14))
 (via (at 146.48 109.26) (size 0.6) (drill 0.3) (layers "F.Cu" "B.Cu") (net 14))
 (segment (start 146.8035 108.9365) (end 161.59075 108.9365) (width 0.2) (layer "B.Cu") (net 14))
 (segment (start 164.45425 111.8) (end 171.55625 111.8) (width 0.2) (layer "B.Cu") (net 14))
 (segment (start 161.59075 108.9365) (end 164.45425 111.8) (width 0.2) (layer "B.Cu") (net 14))
 (segment (start 146.48 109.26) (end 146.8035 108.9365) (width 0.2) (layer "B.Cu") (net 14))
 (segment (start 144.28 101.93075) (end 144.743 102.39375) (width 0.2) (layer "F.Cu") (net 5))
 (segment (start 144.28 101.35) (end 144.28 101.93075) (width 0.2) (layer "F.Cu") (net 5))
 (via (at 144.743 102.39375) (size 0.6) (drill 0.3) (layers "F.Cu" "B.Cu") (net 5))
 (segment (start 196.99275 102.99475) (end 198.59 101.3975) (width 0.2) (layer "B.Cu") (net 5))
 (segment (start 143.217 98.36969) (end 143.83969 97.747) (width 0.2) (layer "B.Cu") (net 5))
 (segment (start 187.6674 97.747) (end 192.91515 102.99475) (width 0.2) (layer "B.Cu") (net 5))
 (segment (start 192.91515 102.99475) (end 196.99275 102.99475) (width 0.2) (layer "B.Cu") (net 5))
 (segment (start 143.83969 97.747) (end 187.6674 97.747) (width 0.2) (layer "B.Cu") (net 5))
 (segment (start 143.217 100.86775) (end 143.217 98.36969) (width 0.2) (layer "B.Cu") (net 5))
 (segment (start 144.743 102.39375) (end 143.217 100.86775) (width 0.2) (layer "B.Cu") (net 5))
 (segment (start 195.37125 107.15625) (end 192.88125 107.15625) (width 0.2) (layer "F.Cu") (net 6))
 (segment (start 198.59 103.9375) (end 195.37125 107.15625) (width 0.2) (layer "F.Cu") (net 6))
 (via (at 192.88125 107.15625) (size 0.6) (drill 0.3) (layers "F.Cu" "B.Cu") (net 6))
 (segment (start 192.88125 107.15625) (end 154.78125 107.15625) (width 0.2) (layer "B.Cu") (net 6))
 (segment (start 154.78125 107.15625) (end 146.435 98.81) (width 0.2) (layer "B.Cu") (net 6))
 (segment (start 146.435 98.81) (end 144.28 98.81) (width 0.2) (layer "B.Cu") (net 6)))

